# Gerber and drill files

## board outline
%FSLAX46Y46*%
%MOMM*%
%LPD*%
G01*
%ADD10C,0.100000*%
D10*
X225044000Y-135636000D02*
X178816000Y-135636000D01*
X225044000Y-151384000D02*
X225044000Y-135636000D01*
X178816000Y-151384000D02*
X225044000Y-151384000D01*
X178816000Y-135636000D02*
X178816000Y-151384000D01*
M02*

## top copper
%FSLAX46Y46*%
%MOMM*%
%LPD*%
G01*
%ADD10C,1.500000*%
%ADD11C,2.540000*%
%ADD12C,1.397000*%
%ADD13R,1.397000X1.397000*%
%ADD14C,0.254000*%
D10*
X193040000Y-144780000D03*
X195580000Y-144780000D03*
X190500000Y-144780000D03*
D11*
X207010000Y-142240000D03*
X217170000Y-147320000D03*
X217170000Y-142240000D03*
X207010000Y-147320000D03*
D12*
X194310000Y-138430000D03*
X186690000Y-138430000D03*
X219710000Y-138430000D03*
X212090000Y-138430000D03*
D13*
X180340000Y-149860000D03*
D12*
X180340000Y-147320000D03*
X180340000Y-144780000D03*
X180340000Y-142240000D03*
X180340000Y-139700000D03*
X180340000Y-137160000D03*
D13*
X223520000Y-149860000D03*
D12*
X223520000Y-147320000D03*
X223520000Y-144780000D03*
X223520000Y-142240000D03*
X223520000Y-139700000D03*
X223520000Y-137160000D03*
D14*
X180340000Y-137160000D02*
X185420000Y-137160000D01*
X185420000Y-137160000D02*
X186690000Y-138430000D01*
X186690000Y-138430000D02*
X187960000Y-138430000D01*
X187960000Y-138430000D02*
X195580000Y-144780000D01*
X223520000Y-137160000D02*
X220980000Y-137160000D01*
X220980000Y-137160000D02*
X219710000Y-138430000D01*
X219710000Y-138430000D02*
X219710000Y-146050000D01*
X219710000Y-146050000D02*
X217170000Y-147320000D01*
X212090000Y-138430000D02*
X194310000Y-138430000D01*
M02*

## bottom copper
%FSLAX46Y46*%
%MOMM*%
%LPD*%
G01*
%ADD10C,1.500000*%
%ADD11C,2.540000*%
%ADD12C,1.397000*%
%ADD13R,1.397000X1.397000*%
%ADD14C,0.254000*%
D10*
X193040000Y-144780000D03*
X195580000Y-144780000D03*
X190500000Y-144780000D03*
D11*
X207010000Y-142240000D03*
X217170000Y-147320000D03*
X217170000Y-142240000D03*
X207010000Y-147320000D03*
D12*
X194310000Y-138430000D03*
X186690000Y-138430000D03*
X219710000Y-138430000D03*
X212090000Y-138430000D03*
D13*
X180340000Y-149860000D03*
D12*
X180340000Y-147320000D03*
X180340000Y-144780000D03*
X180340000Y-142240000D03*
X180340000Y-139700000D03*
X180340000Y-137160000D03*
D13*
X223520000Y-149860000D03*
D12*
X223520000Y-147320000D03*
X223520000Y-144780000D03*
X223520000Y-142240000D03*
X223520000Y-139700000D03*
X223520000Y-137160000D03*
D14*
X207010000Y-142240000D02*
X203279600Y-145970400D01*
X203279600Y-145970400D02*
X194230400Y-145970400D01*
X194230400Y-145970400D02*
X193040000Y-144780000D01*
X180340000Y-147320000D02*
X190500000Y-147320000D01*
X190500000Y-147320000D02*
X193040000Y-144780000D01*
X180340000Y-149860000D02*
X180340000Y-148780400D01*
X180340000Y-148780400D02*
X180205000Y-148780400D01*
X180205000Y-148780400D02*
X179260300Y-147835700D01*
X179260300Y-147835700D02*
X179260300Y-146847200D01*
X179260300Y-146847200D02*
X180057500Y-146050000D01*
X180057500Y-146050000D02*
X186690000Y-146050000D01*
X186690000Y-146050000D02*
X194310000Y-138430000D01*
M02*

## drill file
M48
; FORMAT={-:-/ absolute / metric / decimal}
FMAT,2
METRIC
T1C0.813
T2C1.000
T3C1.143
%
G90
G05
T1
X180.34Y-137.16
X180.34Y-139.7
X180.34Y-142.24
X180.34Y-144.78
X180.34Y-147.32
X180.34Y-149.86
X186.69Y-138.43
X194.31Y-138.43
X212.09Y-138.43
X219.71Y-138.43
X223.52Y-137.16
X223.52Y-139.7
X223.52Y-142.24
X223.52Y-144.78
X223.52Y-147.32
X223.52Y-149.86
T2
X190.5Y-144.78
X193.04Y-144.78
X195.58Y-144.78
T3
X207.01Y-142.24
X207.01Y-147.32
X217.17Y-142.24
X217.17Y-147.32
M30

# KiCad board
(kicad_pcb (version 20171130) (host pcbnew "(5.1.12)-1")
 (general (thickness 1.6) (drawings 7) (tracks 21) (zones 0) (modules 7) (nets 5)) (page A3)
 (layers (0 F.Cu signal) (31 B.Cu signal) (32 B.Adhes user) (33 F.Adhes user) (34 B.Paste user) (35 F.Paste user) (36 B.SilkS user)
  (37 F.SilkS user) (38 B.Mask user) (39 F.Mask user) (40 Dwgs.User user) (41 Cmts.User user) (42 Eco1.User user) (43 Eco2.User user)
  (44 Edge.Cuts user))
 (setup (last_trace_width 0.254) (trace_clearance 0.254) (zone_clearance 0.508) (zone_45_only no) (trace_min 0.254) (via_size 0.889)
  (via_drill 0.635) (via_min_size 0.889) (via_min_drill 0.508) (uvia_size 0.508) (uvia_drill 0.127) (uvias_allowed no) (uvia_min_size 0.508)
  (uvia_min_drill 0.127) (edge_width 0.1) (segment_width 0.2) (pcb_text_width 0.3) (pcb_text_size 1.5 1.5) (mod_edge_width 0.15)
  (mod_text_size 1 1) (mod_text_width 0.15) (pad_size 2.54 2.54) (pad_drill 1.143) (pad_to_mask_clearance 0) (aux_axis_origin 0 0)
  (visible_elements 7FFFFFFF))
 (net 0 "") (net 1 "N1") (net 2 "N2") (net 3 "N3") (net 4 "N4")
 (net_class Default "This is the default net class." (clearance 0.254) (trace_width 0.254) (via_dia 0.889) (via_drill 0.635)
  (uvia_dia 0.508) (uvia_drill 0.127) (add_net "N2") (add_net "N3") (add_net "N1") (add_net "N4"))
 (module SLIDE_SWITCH (layer F.Cu) (at 193.04 144.78)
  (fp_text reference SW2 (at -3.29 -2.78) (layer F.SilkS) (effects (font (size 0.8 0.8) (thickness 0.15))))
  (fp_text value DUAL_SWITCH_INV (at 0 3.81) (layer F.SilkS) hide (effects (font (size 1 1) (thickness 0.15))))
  (pad 2 thru_hole circle (at 0 0) (size 1.5 1.5) (drill 1) (layers *.Cu *.Mask F.SilkS) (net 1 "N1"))
  (pad 1 thru_hole circle (at 2.54 0) (size 1.5 1.5) (drill 1) (layers *.Cu *.Mask F.SilkS) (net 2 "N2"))
  (pad 3 thru_hole circle (at -2.54 0) (size 1.5 1.5) (drill 1) (layers *.Cu *.Mask F.SilkS)))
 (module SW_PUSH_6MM (layer F.Cu) (at 212.09 144.78) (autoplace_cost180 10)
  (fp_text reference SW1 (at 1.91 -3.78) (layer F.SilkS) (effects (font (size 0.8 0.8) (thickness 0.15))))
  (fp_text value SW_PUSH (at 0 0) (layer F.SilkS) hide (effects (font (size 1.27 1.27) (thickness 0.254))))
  (pad 1 thru_hole circle (at -5.08 -2.54) (size 2.54 2.54) (drill 1.143) (layers *.Cu *.Mask F.SilkS) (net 1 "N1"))
  (pad 2 thru_hole circle (at 5.08 2.54) (size 2.54 2.54) (drill 1.143) (layers *.Cu *.Mask F.SilkS) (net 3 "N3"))
  (pad 4 thru_hole circle (at 5.08 -2.54) (size 2.54 2.54) (drill 1.143) (layers *.Cu *.Mask F.SilkS))
  (pad 5 thru_hole circle (at -5.08 2.54) (size 2.54 2.54) (drill 1.143) (layers *.Cu *.Mask F.SilkS)))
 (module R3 (layer F.Cu) (at 190.5 138.43 180) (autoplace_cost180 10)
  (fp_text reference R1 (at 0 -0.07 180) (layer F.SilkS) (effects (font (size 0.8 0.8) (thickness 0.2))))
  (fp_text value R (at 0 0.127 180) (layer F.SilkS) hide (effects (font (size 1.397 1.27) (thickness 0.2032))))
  (pad 1 thru_hole circle (at -3.81 0 180) (size 1.397 1.397) (drill 0.8128) (layers *.Cu *.Mask F.SilkS) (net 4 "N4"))
  (pad 2 thru_hole circle (at 3.81 0 180) (size 1.397 1.397) (drill 0.8128) (layers *.Cu *.Mask F.SilkS) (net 2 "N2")))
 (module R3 (layer F.Cu) (at 215.9 138.43 180) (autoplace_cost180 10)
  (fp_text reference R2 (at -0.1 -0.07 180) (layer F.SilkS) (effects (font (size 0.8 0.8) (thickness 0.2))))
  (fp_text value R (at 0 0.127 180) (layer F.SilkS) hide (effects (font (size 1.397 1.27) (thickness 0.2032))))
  (pad 1 thru_hole circle (at -3.81 0 180) (size 1.397 1.397) (drill 0.8128) (layers *.Cu *.Mask F.SilkS) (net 3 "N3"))
  (pad 2 thru_hole circle (at 3.81 0 180) (size 1.397 1.397) (drill 0.8128) (layers *.Cu *.Mask F.SilkS) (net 4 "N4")))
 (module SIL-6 (layer F.Cu) (at 180.34 143.51 90)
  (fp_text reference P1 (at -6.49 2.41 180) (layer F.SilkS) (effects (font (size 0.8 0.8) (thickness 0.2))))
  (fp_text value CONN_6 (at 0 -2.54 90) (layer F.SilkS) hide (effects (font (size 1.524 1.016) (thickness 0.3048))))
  (pad 1 thru_hole rect (at -6.35 0 90) (size 1.397 1.397) (drill 0.8128) (layers *.Cu *.Mask F.SilkS) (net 4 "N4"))
  (pad 2 thru_hole circle (at -3.81 0 90) (size 1.397 1.397) (drill 0.8128) (layers *.Cu *.Mask F.SilkS) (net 1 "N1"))
  (pad 3 thru_hole circle (at -1.27 0 90) (size 1.397 1.397) (drill 0.8128) (layers *.Cu *.Mask F.SilkS))
  (pad 4 thru_hole circle (at 1.27 0 90) (size 1.397 1.397) (drill 0.8128) (layers *.Cu *.Mask F.SilkS))
  (pad 5 thru_hole circle (at 3.81 0 90) (size 1.397 1.397) (drill 0.8128) (layers *.Cu *.Mask F.SilkS))
  (pad 6 thru_hole circle (at 6.35 0 90) (size 1.397 1.397) (drill 0.8128) (layers *.Cu *.Mask F.SilkS) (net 2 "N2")))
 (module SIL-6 (layer F.Cu) (at 223.52 143.51 90)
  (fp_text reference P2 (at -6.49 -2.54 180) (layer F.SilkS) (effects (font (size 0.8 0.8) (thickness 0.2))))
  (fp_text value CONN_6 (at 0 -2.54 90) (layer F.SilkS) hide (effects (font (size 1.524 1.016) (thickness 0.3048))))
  (pad 1 thru_hole rect (at -6.35 0 90) (size 1.397 1.397) (drill 0.8128) (layers *.Cu *.Mask F.SilkS))
  (pad 2 thru_hole circle (at -3.81 0 90) (size 1.397 1.397) (drill 0.8128) (layers *.Cu *.Mask F.SilkS))
  (pad 3 thru_hole circle (at -1.27 0 90) (size 1.397 1.397) (drill 0.8128) (layers *.Cu *.Mask F.SilkS))
  (pad 4 thru_hole circle (at 1.27 0 90) (size 1.397 1.397) (drill 0.8128) (layers *.Cu *.Mask F.SilkS))
  (pad 5 thru_hole circle (at 3.81 0 90) (size 1.397 1.397) (drill 0.8128) (layers *.Cu *.Mask F.SilkS))
  (pad 6 thru_hole circle (at 6.35 0 90) (size 1.397 1.397) (drill 0.8128) (layers *.Cu *.Mask F.SilkS) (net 3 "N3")))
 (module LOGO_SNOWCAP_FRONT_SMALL (layer F.Cu) (at 184.8 144 90)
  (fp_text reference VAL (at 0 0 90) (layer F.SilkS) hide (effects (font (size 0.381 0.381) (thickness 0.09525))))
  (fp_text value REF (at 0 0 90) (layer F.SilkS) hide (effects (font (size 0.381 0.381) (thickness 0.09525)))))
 (gr_line (start 225.044 135.636) (end 178.816 135.636) (angle 90) (layer Edge.Cuts) (width 0.1))
 (gr_line (start 225.044 151.384) (end 225.044 135.636) (angle 90) (layer Edge.Cuts) (width 0.1))
 (gr_line (start 178.816 151.384) (end 225.044 151.384) (angle 90) (layer Edge.Cuts) (width 0.1))
 (gr_line (start 178.816 135.636) (end 178.816 151.384) (angle 90) (layer Edge.Cuts) (width 0.1))
 (segment (start 180.34 137.16) (end 185.42 137.16) (width 0.254) (layer F.Cu) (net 2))
 (segment (start 185.42 137.16) (end 186.69 138.43) (width 0.254) (layer F.Cu) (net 2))
 (segment (start 186.69 138.43) (end 187.96 138.43) (width 0.254) (layer F.Cu) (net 2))
 (segment (start 187.96 138.43) (end 195.58 144.78) (width 0.254) (layer F.Cu) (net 2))
 (segment (start 223.52 137.16) (end 220.98 137.16) (width 0.254) (layer F.Cu) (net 3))
 (segment (start 220.98 137.16) (end 219.71 138.43) (width 0.254) (layer F.Cu) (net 3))
 (segment (start 219.71 138.43) (end 219.71 146.05) (width 0.254) (layer F.Cu) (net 3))
 (segment (start 219.71 146.05) (end 217.17 147.32) (width 0.254) (layer F.Cu) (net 3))
 (segment (start 207.01 142.24) (end 203.2796 145.9704) (width 0.254) (layer B.Cu) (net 1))
 (segment (start 203.2796 145.9704) (end 194.2304 145.9704) (width 0.254) (layer B.Cu) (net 1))
 (segment (start 194.2304 145.9704) (end 193.04 144.78) (width 0.254) (layer B.Cu) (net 1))
 (segment (start 180.34 147.32) (end 190.5 147.32) (width 0.254) (layer B.Cu) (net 1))
 (segment (start 190.5 147.32) (end 193.04 144.78) (width 0.254) (layer B.Cu) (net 1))
 (segment (start 212.09 138.43) (end 194.31 138.43) (width 0.254) (layer F.Cu) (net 4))
 (segment (start 180.34 149.86) (end 180.34 148.7804) (width 0.254) (layer B.Cu) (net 4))
 (segment (start 180.34 148.7804) (end 180.205 148.7804) (width 0.254) (layer B.Cu) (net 4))
 (segment (start 180.205 148.7804) (end 179.2603 147.8357) (width 0.254) (layer B.Cu) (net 4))
 (segment (start 179.2603 147.8357) (end 179.2603 146.8472) (width 0.254) (layer B.Cu) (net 4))
 (segment (start 179.2603 146.8472) (end 180.0575 146.05) (width 0.254) (layer B.Cu) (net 4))
 (segment (start 180.0575 146.05) (end 186.69 146.05) (width 0.254) (layer B.Cu) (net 4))
 (segment (start 186.69 146.05) (end 194.31 138.43) (width 0.254) (layer B.Cu) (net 4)))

